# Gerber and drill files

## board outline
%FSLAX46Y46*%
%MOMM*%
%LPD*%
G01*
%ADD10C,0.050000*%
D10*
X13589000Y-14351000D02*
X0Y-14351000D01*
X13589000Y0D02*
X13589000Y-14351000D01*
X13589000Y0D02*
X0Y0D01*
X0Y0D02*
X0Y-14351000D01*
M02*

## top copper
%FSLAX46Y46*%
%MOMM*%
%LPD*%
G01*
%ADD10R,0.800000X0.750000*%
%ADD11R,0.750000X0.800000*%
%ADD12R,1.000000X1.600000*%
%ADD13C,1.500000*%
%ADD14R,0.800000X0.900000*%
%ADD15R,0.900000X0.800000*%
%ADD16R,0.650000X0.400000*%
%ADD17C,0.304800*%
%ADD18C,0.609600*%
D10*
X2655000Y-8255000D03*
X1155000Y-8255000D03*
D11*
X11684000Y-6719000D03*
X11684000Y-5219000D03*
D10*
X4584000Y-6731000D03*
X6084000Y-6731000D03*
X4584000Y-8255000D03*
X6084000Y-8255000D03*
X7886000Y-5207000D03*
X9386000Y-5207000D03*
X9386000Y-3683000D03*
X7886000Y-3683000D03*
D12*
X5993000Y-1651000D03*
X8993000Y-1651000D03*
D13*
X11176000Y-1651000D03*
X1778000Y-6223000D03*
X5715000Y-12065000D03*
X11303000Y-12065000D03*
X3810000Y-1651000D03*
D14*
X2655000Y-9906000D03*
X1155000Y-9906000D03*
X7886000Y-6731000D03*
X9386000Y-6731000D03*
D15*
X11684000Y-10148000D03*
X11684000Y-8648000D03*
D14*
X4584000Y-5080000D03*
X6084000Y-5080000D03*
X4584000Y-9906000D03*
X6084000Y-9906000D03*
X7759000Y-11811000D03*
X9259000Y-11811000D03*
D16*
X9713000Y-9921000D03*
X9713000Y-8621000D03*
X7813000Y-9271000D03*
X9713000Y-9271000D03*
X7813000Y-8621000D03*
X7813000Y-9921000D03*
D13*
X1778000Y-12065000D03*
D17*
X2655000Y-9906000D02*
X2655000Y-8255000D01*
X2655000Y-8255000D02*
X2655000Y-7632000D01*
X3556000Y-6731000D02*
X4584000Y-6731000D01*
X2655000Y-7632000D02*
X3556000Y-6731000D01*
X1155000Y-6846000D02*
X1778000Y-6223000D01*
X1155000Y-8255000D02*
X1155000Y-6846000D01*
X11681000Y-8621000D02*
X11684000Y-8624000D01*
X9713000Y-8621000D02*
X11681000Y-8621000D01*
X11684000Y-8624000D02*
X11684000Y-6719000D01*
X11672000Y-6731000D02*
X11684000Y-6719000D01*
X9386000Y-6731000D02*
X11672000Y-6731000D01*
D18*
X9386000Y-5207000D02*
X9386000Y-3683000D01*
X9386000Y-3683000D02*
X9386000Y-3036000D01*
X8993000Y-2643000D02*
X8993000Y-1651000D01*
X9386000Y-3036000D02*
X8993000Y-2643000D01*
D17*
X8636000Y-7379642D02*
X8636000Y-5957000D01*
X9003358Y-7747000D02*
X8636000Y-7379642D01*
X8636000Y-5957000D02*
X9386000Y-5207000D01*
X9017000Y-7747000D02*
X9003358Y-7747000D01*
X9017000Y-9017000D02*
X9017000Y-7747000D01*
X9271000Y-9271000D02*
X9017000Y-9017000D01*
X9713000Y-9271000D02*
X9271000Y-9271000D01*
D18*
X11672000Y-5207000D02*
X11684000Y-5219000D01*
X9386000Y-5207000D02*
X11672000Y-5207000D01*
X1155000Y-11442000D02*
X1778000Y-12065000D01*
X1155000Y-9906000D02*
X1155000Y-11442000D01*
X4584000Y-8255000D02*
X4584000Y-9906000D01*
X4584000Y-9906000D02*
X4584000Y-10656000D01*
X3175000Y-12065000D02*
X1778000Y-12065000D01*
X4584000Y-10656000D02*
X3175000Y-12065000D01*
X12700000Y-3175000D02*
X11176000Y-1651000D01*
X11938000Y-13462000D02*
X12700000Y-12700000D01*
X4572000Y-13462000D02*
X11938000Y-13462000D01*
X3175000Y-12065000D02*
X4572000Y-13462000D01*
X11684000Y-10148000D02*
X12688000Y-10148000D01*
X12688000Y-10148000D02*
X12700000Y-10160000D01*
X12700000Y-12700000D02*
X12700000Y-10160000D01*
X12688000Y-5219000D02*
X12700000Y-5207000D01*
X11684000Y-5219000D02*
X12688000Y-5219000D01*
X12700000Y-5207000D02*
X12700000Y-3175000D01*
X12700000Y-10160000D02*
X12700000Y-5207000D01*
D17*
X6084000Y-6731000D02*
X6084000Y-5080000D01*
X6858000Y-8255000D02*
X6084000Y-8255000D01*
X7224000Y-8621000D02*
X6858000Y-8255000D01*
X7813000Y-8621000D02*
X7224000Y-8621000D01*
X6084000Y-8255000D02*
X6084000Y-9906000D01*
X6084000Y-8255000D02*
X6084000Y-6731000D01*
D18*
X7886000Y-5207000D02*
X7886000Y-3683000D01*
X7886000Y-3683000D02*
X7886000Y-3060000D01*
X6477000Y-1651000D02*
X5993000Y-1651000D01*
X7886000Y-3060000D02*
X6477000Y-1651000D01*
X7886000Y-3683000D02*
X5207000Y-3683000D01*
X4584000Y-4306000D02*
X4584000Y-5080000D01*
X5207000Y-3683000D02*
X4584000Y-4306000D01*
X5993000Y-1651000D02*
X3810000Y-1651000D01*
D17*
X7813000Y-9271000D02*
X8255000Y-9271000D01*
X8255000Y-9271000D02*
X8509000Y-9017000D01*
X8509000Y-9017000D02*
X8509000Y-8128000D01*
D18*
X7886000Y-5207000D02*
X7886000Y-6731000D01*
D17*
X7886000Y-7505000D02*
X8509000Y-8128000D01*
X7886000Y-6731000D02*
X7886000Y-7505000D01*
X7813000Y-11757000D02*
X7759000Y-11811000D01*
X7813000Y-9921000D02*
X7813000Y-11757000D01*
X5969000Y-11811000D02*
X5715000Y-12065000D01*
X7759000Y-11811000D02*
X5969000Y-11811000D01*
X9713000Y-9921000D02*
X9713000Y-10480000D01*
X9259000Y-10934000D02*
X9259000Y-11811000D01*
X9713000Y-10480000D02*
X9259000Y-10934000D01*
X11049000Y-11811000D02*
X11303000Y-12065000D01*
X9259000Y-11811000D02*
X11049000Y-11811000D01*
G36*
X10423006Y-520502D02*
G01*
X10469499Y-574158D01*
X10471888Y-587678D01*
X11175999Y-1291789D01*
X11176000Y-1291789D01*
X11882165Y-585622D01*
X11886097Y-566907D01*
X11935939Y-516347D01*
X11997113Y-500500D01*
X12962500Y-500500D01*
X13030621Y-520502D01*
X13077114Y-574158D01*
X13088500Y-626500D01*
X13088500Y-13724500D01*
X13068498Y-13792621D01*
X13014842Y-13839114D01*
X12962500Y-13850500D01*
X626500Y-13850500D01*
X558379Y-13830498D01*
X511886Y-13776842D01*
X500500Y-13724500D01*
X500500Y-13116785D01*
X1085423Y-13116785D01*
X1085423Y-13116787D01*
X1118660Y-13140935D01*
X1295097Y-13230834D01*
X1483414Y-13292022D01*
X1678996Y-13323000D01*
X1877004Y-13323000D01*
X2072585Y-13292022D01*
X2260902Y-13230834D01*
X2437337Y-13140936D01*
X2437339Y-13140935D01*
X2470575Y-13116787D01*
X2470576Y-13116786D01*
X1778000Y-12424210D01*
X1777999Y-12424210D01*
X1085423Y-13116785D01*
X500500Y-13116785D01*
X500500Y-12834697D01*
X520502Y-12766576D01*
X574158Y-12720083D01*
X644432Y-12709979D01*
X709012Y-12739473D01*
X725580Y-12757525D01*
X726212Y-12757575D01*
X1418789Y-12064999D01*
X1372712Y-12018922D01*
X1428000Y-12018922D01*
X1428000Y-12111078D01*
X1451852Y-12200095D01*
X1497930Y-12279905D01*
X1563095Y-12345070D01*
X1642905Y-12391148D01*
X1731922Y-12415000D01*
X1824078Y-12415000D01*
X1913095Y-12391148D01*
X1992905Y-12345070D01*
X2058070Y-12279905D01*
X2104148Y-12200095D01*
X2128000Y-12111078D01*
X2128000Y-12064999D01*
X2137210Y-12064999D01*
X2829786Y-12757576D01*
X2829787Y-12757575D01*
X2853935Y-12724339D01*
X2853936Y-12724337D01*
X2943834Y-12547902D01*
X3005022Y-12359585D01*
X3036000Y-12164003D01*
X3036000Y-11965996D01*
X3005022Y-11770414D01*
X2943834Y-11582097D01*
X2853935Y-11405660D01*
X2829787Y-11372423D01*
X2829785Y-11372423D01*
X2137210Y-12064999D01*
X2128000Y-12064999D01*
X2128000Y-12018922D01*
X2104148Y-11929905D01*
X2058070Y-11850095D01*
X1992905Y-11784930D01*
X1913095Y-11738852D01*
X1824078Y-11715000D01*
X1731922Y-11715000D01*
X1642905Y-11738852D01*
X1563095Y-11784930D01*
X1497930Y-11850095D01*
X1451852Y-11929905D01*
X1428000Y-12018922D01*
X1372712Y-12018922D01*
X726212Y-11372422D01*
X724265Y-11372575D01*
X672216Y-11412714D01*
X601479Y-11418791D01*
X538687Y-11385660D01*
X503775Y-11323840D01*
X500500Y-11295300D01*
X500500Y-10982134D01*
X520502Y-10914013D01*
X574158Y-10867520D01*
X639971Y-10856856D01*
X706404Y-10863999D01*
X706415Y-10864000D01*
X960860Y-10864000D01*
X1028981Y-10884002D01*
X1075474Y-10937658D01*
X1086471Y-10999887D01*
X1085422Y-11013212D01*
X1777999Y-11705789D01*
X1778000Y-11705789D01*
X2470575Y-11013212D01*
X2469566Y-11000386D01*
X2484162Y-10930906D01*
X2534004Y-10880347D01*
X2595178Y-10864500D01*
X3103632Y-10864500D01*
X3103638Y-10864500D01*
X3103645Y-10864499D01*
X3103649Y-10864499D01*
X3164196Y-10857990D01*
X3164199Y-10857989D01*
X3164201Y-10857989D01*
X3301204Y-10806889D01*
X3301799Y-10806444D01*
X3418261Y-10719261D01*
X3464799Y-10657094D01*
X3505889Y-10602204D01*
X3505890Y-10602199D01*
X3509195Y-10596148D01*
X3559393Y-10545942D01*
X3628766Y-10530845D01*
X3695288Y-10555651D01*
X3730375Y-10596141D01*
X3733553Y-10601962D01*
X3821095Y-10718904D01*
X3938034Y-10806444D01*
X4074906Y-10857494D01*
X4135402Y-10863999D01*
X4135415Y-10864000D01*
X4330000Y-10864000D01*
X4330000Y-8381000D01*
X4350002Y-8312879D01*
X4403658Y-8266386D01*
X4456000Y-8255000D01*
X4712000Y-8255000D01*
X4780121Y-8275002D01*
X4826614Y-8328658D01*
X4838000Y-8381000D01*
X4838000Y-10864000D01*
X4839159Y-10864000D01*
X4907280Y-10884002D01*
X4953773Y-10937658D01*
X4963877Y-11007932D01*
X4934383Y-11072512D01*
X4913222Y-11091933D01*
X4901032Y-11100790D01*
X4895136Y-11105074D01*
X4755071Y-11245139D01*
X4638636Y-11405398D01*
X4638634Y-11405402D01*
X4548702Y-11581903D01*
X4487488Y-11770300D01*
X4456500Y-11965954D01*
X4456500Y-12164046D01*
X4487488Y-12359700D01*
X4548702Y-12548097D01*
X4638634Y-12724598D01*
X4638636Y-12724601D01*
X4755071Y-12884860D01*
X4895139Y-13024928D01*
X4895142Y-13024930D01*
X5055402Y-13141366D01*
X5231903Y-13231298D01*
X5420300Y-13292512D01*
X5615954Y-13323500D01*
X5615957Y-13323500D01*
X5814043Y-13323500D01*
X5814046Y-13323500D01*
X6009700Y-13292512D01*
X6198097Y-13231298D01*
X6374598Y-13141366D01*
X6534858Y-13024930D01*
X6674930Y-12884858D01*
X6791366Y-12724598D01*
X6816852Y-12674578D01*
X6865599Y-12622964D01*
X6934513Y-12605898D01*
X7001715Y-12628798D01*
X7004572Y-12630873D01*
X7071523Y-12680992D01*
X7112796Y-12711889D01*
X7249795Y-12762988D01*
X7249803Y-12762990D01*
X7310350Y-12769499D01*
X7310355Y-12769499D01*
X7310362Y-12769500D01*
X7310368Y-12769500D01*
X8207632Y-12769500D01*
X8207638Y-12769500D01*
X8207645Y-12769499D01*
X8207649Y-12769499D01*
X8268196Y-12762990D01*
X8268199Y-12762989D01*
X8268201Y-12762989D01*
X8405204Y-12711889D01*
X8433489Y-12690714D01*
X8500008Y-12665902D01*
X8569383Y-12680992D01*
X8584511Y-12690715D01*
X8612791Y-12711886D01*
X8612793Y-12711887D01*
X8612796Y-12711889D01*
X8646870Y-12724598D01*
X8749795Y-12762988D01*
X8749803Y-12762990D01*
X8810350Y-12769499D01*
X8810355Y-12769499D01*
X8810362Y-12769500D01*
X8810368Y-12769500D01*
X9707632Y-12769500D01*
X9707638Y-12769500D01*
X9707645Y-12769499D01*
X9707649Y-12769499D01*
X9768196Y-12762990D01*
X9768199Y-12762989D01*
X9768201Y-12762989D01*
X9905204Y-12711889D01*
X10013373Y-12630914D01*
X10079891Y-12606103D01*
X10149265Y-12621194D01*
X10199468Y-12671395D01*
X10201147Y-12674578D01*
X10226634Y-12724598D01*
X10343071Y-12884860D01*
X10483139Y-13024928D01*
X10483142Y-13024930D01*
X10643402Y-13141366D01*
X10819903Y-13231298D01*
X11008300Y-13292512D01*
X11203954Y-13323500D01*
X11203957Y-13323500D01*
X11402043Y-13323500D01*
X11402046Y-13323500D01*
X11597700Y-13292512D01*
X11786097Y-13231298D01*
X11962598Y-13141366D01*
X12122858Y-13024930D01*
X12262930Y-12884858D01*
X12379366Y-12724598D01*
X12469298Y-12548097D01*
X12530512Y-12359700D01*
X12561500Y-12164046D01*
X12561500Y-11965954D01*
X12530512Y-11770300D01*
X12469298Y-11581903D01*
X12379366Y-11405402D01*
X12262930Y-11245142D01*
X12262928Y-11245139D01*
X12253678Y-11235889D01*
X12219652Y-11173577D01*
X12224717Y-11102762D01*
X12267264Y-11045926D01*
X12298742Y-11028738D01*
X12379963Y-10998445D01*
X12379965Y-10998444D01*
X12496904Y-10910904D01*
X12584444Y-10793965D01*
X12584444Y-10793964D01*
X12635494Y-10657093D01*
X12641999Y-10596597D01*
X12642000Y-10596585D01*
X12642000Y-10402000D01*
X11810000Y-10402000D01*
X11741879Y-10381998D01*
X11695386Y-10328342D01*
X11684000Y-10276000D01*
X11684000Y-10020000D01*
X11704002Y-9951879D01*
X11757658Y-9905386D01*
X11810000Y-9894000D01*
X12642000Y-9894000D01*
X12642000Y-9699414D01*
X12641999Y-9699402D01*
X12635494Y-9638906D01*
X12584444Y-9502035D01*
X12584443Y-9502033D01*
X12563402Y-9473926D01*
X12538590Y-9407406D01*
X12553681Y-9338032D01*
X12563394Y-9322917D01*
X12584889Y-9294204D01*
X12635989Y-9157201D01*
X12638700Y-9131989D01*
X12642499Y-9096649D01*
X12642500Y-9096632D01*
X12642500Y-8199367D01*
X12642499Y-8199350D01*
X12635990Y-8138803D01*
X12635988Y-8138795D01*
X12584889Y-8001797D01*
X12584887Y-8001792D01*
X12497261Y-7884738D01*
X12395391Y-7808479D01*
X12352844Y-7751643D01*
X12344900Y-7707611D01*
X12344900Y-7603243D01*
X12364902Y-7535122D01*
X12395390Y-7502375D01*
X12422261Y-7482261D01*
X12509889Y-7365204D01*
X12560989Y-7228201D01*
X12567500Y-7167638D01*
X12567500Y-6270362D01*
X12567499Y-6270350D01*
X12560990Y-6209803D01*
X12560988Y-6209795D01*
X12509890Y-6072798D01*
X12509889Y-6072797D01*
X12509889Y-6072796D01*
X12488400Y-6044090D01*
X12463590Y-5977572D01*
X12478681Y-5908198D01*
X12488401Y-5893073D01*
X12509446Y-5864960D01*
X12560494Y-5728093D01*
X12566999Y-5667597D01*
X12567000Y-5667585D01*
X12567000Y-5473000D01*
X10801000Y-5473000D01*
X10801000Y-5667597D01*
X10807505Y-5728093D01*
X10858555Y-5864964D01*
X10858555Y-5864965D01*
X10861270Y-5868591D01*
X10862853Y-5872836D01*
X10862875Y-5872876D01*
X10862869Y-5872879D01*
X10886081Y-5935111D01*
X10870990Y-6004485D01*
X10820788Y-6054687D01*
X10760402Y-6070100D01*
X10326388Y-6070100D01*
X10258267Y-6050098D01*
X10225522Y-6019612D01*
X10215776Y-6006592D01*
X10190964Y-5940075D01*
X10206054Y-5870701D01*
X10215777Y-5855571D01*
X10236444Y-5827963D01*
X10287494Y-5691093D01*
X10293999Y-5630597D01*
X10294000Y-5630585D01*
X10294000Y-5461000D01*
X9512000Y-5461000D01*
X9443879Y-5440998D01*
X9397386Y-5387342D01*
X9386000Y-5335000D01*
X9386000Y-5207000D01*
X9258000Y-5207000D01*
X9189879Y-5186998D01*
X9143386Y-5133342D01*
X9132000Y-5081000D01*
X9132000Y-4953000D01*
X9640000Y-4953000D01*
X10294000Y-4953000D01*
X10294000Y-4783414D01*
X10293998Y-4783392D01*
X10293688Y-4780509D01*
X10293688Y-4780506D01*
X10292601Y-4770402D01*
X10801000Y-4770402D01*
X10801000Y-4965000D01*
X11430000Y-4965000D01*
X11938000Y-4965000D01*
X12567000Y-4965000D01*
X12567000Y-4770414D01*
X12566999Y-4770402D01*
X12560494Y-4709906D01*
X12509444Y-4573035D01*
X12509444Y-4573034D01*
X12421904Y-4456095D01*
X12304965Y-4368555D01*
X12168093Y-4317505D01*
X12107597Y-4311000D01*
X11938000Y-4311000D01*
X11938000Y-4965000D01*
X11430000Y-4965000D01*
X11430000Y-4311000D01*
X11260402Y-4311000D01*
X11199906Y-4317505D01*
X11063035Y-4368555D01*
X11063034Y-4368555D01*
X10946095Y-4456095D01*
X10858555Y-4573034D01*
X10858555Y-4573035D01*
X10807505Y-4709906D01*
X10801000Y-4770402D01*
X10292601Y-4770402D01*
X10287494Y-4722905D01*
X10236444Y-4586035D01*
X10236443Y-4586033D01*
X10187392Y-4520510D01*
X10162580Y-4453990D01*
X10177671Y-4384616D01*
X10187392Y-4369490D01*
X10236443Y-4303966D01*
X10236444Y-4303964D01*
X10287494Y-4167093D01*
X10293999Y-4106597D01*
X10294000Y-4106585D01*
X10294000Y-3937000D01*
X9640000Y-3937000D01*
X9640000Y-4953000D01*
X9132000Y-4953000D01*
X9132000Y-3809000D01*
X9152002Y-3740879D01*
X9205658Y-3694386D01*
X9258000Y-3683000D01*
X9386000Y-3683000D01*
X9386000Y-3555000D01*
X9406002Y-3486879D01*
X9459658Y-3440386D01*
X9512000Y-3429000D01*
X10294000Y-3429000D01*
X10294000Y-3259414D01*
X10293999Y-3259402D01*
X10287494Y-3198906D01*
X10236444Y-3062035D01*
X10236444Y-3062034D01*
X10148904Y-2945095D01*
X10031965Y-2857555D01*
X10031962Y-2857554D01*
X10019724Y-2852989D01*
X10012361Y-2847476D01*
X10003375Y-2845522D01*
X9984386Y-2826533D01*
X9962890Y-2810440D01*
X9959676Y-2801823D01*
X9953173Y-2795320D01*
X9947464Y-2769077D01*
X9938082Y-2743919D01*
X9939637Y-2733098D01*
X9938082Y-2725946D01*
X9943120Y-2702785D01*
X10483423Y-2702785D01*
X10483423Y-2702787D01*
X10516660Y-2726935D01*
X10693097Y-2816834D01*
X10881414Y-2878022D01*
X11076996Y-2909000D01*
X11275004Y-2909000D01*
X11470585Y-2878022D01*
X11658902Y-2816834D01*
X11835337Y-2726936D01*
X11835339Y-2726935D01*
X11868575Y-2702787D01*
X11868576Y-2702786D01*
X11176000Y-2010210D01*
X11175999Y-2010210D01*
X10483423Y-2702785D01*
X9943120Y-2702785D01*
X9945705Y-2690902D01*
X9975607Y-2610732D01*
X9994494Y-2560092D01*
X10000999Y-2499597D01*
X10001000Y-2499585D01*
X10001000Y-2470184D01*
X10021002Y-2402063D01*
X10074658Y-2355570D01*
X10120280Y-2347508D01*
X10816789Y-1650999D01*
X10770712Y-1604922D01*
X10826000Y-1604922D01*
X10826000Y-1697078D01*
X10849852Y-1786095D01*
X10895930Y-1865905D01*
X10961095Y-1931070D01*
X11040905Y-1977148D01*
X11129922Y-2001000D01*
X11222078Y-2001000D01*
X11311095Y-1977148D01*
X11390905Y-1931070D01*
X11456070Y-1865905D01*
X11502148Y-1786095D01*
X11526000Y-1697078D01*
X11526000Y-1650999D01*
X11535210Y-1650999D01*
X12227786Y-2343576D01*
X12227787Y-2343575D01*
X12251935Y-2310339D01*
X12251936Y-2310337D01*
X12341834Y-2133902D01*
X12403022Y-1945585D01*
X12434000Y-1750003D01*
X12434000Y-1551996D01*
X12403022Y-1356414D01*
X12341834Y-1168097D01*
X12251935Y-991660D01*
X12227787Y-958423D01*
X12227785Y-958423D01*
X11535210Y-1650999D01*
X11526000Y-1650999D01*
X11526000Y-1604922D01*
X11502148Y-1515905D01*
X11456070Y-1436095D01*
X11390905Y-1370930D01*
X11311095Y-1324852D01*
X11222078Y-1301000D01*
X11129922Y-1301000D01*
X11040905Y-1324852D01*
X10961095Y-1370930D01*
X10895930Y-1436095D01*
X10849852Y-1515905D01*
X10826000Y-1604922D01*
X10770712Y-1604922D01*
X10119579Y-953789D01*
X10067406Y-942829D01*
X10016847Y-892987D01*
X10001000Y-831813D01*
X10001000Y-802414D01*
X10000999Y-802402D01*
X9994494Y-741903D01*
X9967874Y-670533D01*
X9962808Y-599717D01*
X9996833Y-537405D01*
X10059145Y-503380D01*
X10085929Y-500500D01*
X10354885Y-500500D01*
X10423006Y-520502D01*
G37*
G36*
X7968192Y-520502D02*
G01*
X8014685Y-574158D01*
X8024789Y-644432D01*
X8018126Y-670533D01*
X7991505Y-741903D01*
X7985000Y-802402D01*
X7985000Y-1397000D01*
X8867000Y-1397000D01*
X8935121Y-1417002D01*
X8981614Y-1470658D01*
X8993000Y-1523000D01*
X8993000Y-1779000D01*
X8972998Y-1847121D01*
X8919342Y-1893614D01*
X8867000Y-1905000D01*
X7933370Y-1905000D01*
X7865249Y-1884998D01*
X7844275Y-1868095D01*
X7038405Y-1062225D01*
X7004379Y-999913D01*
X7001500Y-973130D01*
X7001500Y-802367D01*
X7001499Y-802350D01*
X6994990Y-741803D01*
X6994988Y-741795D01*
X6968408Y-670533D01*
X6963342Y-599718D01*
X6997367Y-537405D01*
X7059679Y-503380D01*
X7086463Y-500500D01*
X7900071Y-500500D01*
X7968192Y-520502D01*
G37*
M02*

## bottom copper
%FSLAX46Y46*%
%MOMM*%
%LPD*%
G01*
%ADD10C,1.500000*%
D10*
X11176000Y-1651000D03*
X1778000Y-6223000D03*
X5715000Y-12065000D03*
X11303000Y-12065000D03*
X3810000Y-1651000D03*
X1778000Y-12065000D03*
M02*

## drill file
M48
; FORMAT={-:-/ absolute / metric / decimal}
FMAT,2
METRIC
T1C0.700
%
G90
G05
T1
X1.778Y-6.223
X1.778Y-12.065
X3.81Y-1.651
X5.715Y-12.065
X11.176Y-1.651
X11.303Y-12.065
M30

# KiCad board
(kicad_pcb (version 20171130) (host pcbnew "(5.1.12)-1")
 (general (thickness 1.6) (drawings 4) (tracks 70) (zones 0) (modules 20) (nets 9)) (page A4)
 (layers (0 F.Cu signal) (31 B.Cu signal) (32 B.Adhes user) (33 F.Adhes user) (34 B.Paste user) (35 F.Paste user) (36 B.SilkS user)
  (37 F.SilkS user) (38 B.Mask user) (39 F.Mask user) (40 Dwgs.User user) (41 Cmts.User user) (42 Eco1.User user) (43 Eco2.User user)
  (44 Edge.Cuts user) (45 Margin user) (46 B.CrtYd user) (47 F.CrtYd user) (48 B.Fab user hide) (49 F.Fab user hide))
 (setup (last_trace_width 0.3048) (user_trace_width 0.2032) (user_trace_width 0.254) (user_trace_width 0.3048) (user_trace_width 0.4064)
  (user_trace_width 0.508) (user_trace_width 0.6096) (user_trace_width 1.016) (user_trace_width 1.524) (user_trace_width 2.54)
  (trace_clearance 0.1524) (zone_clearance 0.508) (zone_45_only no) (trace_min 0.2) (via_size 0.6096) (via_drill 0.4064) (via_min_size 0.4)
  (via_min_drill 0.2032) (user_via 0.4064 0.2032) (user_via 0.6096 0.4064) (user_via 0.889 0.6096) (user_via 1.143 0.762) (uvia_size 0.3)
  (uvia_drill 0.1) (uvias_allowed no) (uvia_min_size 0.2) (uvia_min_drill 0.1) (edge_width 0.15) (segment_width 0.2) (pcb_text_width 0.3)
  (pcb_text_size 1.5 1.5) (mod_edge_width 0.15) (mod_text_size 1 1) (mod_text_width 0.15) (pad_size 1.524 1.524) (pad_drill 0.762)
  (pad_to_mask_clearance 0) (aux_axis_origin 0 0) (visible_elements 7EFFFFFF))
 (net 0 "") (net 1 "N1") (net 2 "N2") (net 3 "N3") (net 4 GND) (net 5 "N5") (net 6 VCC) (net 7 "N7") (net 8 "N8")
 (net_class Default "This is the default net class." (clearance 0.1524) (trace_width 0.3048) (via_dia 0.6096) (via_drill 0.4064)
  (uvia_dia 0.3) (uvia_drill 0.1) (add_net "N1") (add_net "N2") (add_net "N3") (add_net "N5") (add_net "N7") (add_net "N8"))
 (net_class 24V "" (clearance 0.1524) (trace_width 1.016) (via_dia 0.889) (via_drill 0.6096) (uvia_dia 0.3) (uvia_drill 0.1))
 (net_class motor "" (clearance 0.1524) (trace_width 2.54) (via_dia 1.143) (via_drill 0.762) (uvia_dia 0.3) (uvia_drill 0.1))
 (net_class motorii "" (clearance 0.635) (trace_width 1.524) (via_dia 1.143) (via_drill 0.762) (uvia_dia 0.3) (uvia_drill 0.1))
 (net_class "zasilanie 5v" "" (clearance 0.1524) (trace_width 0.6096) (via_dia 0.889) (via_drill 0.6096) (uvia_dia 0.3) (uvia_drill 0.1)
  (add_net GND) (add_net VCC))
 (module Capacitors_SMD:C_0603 (layer F.Cu) (at 1.905 8.255 180)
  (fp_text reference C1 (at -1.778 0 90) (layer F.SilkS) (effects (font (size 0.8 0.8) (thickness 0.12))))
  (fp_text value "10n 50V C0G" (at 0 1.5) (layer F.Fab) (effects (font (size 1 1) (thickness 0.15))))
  (pad 1 smd rect (at -0.75 0 180) (size 0.8 0.75) (layers F.Cu F.Paste F.Mask) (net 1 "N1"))
  (pad 2 smd rect (at 0.75 0 180) (size 0.8 0.75) (layers F.Cu F.Paste F.Mask) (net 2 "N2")))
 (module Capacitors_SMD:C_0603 (layer F.Cu) (at 11.684 5.969 90)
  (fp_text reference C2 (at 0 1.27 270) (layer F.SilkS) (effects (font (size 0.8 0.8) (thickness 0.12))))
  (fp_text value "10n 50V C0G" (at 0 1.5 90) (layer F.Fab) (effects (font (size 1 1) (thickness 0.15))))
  (pad 1 smd rect (at -0.75 0 90) (size 0.8 0.75) (layers F.Cu F.Paste F.Mask) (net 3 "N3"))
  (pad 2 smd rect (at 0.75 0 90) (size 0.8 0.75) (layers F.Cu F.Paste F.Mask) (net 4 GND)))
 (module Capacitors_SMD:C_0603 (layer F.Cu) (at 5.334 6.731 180)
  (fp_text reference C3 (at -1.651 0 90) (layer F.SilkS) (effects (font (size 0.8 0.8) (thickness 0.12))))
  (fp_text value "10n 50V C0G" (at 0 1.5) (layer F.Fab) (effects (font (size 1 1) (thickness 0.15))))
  (pad 2 smd rect (at 0.75 0 180) (size 0.8 0.75) (layers F.Cu F.Paste F.Mask) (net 1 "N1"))
  (pad 1 smd rect (at -0.75 0 180) (size 0.8 0.75) (layers F.Cu F.Paste F.Mask) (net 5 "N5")))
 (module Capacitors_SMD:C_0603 (layer F.Cu) (at 5.334 8.255 180)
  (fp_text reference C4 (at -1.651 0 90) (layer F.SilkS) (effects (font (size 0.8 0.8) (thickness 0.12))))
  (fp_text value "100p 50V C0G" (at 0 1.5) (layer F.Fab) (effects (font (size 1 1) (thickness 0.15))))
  (pad 2 smd rect (at 0.75 0 180) (size 0.8 0.75) (layers F.Cu F.Paste F.Mask) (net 4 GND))
  (pad 1 smd rect (at -0.75 0 180) (size 0.8 0.75) (layers F.Cu F.Paste F.Mask) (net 5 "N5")))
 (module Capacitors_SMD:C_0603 (layer F.Cu) (at 8.636 5.207)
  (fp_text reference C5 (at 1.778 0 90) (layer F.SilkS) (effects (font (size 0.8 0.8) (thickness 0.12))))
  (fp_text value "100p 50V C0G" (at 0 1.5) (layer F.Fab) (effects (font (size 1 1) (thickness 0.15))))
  (pad 1 smd rect (at -0.75 0) (size 0.8 0.75) (layers F.Cu F.Paste F.Mask) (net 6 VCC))
  (pad 2 smd rect (at 0.75 0) (size 0.8 0.75) (layers F.Cu F.Paste F.Mask) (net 4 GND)))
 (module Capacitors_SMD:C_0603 (layer F.Cu) (at 8.636 3.683)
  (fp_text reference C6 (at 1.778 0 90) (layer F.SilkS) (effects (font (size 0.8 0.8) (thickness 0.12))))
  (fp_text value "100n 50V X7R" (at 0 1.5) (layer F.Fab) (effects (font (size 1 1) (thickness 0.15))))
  (pad 2 smd rect (at 0.75 0) (size 0.8 0.75) (layers F.Cu F.Paste F.Mask) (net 4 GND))
  (pad 1 smd rect (at -0.75 0) (size 0.8 0.75) (layers F.Cu F.Paste F.Mask) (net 6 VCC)))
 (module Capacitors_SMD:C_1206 (layer F.Cu) (at 7.493 1.651)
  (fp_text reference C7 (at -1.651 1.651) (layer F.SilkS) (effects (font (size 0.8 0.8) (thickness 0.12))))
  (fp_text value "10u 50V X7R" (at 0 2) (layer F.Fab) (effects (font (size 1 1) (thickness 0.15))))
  (pad 1 smd rect (at -1.5 0) (size 1 1.6) (layers F.Cu F.Paste F.Mask) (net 6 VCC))
  (pad 2 smd rect (at 1.5 0) (size 1 1.6) (layers F.Cu F.Paste F.Mask) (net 4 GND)))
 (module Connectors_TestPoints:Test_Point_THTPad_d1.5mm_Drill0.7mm (layer F.Cu) (at 11.176 1.651)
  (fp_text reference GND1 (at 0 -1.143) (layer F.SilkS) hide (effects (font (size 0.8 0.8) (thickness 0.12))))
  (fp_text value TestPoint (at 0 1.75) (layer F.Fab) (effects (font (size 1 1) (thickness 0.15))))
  (pad 1 thru_hole circle (at 0 0) (size 1.5 1.5) (drill 0.7) (layers *.Cu *.Mask) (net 4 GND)))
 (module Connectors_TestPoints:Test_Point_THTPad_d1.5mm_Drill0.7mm (layer F.Cu) (at 1.778 6.223)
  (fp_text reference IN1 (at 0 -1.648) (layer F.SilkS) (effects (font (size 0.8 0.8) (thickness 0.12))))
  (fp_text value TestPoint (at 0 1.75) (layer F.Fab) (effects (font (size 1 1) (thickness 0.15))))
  (pad 1 thru_hole circle (at 0 0) (size 1.5 1.5) (drill 0.7) (layers *.Cu *.Mask) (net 2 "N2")))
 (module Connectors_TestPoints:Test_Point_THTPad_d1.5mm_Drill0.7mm (layer F.Cu) (at 5.715 12.065)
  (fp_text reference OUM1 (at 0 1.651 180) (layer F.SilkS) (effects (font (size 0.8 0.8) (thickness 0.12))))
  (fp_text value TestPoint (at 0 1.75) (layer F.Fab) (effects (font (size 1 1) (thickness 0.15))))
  (pad 1 thru_hole circle (at 0 0) (size 1.5 1.5) (drill 0.7) (layers *.Cu *.Mask) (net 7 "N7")))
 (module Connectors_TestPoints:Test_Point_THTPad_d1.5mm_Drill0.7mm (layer F.Cu) (at 11.303 12.065)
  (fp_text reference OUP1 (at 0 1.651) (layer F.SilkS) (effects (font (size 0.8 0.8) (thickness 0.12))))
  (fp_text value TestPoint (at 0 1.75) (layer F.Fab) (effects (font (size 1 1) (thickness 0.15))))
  (pad 1 thru_hole circle (at 0 0) (size 1.5 1.5) (drill 0.7) (layers *.Cu *.Mask) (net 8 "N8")))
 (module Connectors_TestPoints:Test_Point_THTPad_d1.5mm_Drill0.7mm (layer F.Cu) (at 3.81 1.651)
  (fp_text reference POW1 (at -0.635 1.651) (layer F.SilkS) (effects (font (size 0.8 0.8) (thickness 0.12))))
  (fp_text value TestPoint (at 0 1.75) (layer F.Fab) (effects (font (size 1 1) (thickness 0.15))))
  (pad 1 thru_hole circle (at 0 0) (size 1.5 1.5) (drill 0.7) (layers *.Cu *.Mask) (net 6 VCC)))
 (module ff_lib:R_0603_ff (layer F.Cu) (at 1.905 9.906 180)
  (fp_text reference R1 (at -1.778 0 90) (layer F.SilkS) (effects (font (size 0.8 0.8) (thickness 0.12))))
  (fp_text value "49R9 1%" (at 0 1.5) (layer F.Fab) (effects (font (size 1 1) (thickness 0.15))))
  (pad 1 smd rect (at -0.75 0 180) (size 0.8 0.9) (layers F.Cu F.Paste F.Mask) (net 1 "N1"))
  (pad 2 smd rect (at 0.75 0 180) (size 0.8 0.9) (layers F.Cu F.Paste F.Mask) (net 4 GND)))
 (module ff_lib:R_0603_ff (layer F.Cu) (at 8.636 6.731)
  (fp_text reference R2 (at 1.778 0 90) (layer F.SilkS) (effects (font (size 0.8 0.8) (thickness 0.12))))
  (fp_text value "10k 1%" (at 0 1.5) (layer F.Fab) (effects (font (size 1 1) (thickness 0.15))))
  (pad 1 smd rect (at -0.75 0) (size 0.8 0.9) (layers F.Cu F.Paste F.Mask) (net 6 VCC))
  (pad 2 smd rect (at 0.75 0) (size 0.8 0.9) (layers F.Cu F.Paste F.Mask) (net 3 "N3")))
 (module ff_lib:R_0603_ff (layer F.Cu) (at 11.684 9.398 270)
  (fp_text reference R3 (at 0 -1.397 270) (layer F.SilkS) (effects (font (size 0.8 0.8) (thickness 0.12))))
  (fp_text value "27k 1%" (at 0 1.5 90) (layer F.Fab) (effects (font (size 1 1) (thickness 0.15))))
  (pad 2 smd rect (at 0.75 0 270) (size 0.8 0.9) (layers F.Cu F.Paste F.Mask) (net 4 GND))
  (pad 1 smd rect (at -0.75 0 270) (size 0.8 0.9) (layers F.Cu F.Paste F.Mask) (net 3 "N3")))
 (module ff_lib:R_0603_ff (layer F.Cu) (at 5.334 5.08)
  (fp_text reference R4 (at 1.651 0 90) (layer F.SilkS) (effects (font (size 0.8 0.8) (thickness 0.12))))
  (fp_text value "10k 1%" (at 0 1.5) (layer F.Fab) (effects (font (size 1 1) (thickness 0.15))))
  (pad 1 smd rect (at -0.75 0) (size 0.8 0.9) (layers F.Cu F.Paste F.Mask) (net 6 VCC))
  (pad 2 smd rect (at 0.75 0) (size 0.8 0.9) (layers F.Cu F.Paste F.Mask) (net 5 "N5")))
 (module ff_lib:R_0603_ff (layer F.Cu) (at 5.334 9.906 180)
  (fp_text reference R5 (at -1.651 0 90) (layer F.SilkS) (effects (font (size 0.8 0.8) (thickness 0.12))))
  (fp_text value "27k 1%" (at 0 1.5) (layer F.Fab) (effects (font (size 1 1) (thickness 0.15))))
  (pad 2 smd rect (at 0.75 0 180) (size 0.8 0.9) (layers F.Cu F.Paste F.Mask) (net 4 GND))
  (pad 1 smd rect (at -0.75 0 180) (size 0.8 0.9) (layers F.Cu F.Paste F.Mask) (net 5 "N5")))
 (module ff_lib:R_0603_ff (layer F.Cu) (at 8.509 11.811 180)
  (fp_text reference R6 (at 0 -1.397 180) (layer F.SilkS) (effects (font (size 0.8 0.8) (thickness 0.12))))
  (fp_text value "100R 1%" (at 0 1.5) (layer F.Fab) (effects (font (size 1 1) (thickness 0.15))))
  (pad 2 smd rect (at 0.75 0 180) (size 0.8 0.9) (layers F.Cu F.Paste F.Mask) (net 7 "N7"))
  (pad 1 smd rect (at -0.75 0 180) (size 0.8 0.9) (layers F.Cu F.Paste F.Mask) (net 8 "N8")))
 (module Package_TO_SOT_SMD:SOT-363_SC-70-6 (layer F.Cu) (at 8.763 9.271 180)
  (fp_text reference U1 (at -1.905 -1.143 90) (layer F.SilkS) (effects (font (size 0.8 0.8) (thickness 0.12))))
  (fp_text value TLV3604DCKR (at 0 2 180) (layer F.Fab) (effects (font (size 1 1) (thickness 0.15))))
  (pad 1 smd rect (at -0.95 -0.65 180) (size 0.65 0.4) (layers F.Cu F.Paste F.Mask) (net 8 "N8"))
  (pad 3 smd rect (at -0.95 0.65 180) (size 0.65 0.4) (layers F.Cu F.Paste F.Mask) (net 3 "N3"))
  (pad 5 smd rect (at 0.95 0 180) (size 0.65 0.4) (layers F.Cu F.Paste F.Mask) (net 6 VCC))
  (pad 2 smd rect (at -0.95 0 180) (size 0.65 0.4) (layers F.Cu F.Paste F.Mask) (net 4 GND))
  (pad 4 smd rect (at 0.95 0.65 180) (size 0.65 0.4) (layers F.Cu F.Paste F.Mask) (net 5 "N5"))
  (pad 6 smd rect (at 0.95 -0.65 180) (size 0.65 0.4) (layers F.Cu F.Paste F.Mask) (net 7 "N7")))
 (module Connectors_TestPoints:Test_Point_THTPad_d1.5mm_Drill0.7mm (layer F.Cu) (at 1.778 12.065)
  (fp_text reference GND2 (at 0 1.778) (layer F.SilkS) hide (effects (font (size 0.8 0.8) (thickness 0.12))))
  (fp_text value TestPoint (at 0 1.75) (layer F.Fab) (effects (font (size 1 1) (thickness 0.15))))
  (pad 1 thru_hole circle (at 0 0) (size 1.5 1.5) (drill 0.7) (layers *.Cu *.Mask) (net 4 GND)))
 (gr_line (start 13.589 14.351) (end 0 14.351) (layer Edge.Cuts) (width 0.05))
 (gr_line (start 13.589 0) (end 13.589 14.351) (layer Edge.Cuts) (width 0.05))
 (gr_line (start 13.589 0) (end 0 0) (layer Edge.Cuts) (width 0.05))
 (gr_line (start 0 0) (end 0 14.351) (layer Edge.Cuts) (width 0.05))
 (segment (start 2.655 9.906) (end 2.655 8.255) (width 0.3048) (layer F.Cu) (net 1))
 (segment (start 2.655 8.255) (end 2.655 7.632) (width 0.3048) (layer F.Cu) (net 1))
 (segment (start 3.556 6.731) (end 4.584 6.731) (width 0.3048) (layer F.Cu) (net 1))
 (segment (start 2.655 7.632) (end 3.556 6.731) (width 0.3048) (layer F.Cu) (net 1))
 (segment (start 1.155 6.846) (end 1.778 6.223) (width 0.3048) (layer F.Cu) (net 2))
 (segment (start 1.155 8.255) (end 1.155 6.846) (width 0.3048) (layer F.Cu) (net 2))
 (segment (start 11.681 8.621) (end 11.684 8.624) (width 0.3048) (layer F.Cu) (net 3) (status 30))
 (segment (start 9.713 8.621) (end 11.681 8.621) (width 0.3048) (layer F.Cu) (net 3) (status 30))
 (segment (start 11.684 8.624) (end 11.684 6.719) (width 0.3048) (layer F.Cu) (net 3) (status 30))
 (segment (start 11.672 6.731) (end 11.684 6.719) (width 0.3048) (layer F.Cu) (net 3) (status 30))
 (segment (start 9.386 6.731) (end 11.672 6.731) (width 0.3048) (layer F.Cu) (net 3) (status 30))
 (segment (start 9.386 5.207) (end 9.386 3.683) (width 0.6096) (layer F.Cu) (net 4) (status 30))
 (segment (start 9.386 3.683) (end 9.386 3.036) (width 0.6096) (layer F.Cu) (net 4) (status 10))
 (segment (start 8.993 2.643) (end 8.993 1.651) (width 0.6096) (layer F.Cu) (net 4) (status 20))
 (segment (start 9.386 3.036) (end 8.993 2.643) (width 0.6096) (layer F.Cu) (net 4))
 (segment (start 8.636 7.379642) (end 8.636 5.957) (width 0.3048) (layer F.Cu) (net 4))
 (segment (start 9.003358 7.747) (end 8.636 7.379642) (width 0.3048) (layer F.Cu) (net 4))
 (segment (start 8.636 5.957) (end 9.386 5.207) (width 0.3048) (layer F.Cu) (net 4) (status 20))
 (segment (start 9.017 7.747) (end 9.003358 7.747) (width 0.3048) (layer F.Cu) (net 4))
 (segment (start 9.017 9.017) (end 9.017 7.747) (width 0.3048) (layer F.Cu) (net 4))
 (segment (start 9.271 9.271) (end 9.017 9.017) (width 0.3048) (layer F.Cu) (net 4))
 (segment (start 9.713 9.271) (end 9.271 9.271) (width 0.3048) (layer F.Cu) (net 4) (status 10))
 (segment (start 11.672 5.207) (end 11.684 5.219) (width 0.6096) (layer F.Cu) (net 4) (status 30))
 (segment (start 9.386 5.207) (end 11.672 5.207) (width 0.6096) (layer F.Cu) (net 4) (status 30))
 (segment (start 1.155 11.442) (end 1.778 12.065) (width 0.6096) (layer F.Cu) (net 4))
 (segment (start 1.155 9.906) (end 1.155 11.442) (width 0.6096) (layer F.Cu) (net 4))
 (segment (start 4.584 8.255) (end 4.584 9.906) (width 0.6096) (layer F.Cu) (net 4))
 (segment (start 4.584 9.906) (end 4.584 10.656) (width 0.6096) (layer F.Cu) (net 4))
 (segment (start 3.175 12.065) (end 1.778 12.065) (width 0.6096) (layer F.Cu) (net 4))
 (segment (start 4.584 10.656) (end 3.175 12.065) (width 0.6096) (layer F.Cu) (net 4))
 (segment (start 12.7 3.175) (end 11.176 1.651) (width 0.6096) (layer F.Cu) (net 4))
 (segment (start 11.938 13.462) (end 12.7 12.7) (width 0.6096) (layer F.Cu) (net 4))
 (segment (start 4.572 13.462) (end 11.938 13.462) (width 0.6096) (layer F.Cu) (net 4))
 (segment (start 3.175 12.065) (end 4.572 13.462) (width 0.6096) (layer F.Cu) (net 4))
 (segment (start 11.684 10.148) (end 12.688 10.148) (width 0.6096) (layer F.Cu) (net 4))
 (segment (start 12.688 10.148) (end 12.7 10.16) (width 0.6096) (layer F.Cu) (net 4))
 (segment (start 12.7 12.7) (end 12.7 10.16) (width 0.6096) (layer F.Cu) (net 4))
 (segment (start 12.688 5.219) (end 12.7 5.207) (width 0.6096) (layer F.Cu) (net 4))
 (segment (start 11.684 5.219) (end 12.688 5.219) (width 0.6096) (layer F.Cu) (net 4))
 (segment (start 12.7 5.207) (end 12.7 3.175) (width 0.6096) (layer F.Cu) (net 4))
 (segment (start 12.7 10.16) (end 12.7 5.207) (width 0.6096) (layer F.Cu) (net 4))
 (segment (start 6.084 6.731) (end 6.084 5.08) (width 0.3048) (layer F.Cu) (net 5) (status 30))
 (segment (start 6.858 8.255) (end 6.084 8.255) (width 0.3048) (layer F.Cu) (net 5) (status 20))
 (segment (start 7.224 8.621) (end 6.858 8.255) (width 0.3048) (layer F.Cu) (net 5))
 (segment (start 7.813 8.621) (end 7.224 8.621) (width 0.3048) (layer F.Cu) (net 5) (status 10))
 (segment (start 6.084 8.255) (end 6.084 9.906) (width 0.3048) (layer F.Cu) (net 5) (status 30))
 (segment (start 6.084 8.255) (end 6.084 6.731) (width 0.3048) (layer F.Cu) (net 5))
 (segment (start 7.886 5.207) (end 7.886 3.683) (width 0.6096) (layer F.Cu) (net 6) (status 30))
 (segment (start 7.886 3.683) (end 7.886 3.06) (width 0.6096) (layer F.Cu) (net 6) (status 10))
 (segment (start 6.477 1.651) (end 5.993 1.651) (width 0.6096) (layer F.Cu) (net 6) (status 30))
 (segment (start 7.886 3.06) (end 6.477 1.651) (width 0.6096) (layer F.Cu) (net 6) (status 20))
 (segment (start 7.886 3.683) (end 5.207 3.683) (width 0.6096) (layer F.Cu) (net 6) (status 10))
 (segment (start 4.584 4.306) (end 4.584 5.08) (width 0.6096) (layer F.Cu) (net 6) (status 20))
 (segment (start 5.207 3.683) (end 4.584 4.306) (width 0.6096) (layer F.Cu) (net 6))
 (segment (start 5.993 1.651) (end 3.81 1.651) (width 0.6096) (layer F.Cu) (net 6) (status 30))
 (segment (start 7.813 9.271) (end 8.255 9.271) (width 0.3048) (layer F.Cu) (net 6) (status 10))
 (segment (start 8.255 9.271) (end 8.509 9.017) (width 0.3048) (layer F.Cu) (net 6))
 (segment (start 8.509 9.017) (end 8.509 8.128) (width 0.3048) (layer F.Cu) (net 6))
 (segment (start 7.886 5.207) (end 7.886 6.731) (width 0.6096) (layer F.Cu) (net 6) (status 30))
 (segment (start 7.886 7.505) (end 8.509 8.128) (width 0.3048) (layer F.Cu) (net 6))
 (segment (start 7.886 6.731) (end 7.886 7.505) (width 0.3048) (layer F.Cu) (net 6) (status 10))
 (segment (start 7.813 11.757) (end 7.759 11.811) (width 0.3048) (layer F.Cu) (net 7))
 (segment (start 7.813 9.921) (end 7.813 11.757) (width 0.3048) (layer F.Cu) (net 7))
 (segment (start 5.969 11.811) (end 5.715 12.065) (width 0.3048) (layer F.Cu) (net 7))
 (segment (start 7.759 11.811) (end 5.969 11.811) (width 0.3048) (layer F.Cu) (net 7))
 (segment (start 9.713 9.921) (end 9.713 10.48) (width 0.3048) (layer F.Cu) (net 8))
 (segment (start 9.259 10.934) (end 9.259 11.811) (width 0.3048) (layer F.Cu) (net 8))
 (segment (start 9.713 10.48) (end 9.259 10.934) (width 0.3048) (layer F.Cu) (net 8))
 (segment (start 11.049 11.811) (end 11.303 12.065) (width 0.3048) (layer F.Cu) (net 8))
 (segment (start 9.259 11.811) (end 11.049 11.811) (width 0.3048) (layer F.Cu) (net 8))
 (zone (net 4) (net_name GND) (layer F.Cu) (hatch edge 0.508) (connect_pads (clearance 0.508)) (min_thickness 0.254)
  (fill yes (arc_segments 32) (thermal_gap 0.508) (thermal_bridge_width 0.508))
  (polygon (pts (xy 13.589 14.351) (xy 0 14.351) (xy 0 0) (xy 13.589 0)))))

